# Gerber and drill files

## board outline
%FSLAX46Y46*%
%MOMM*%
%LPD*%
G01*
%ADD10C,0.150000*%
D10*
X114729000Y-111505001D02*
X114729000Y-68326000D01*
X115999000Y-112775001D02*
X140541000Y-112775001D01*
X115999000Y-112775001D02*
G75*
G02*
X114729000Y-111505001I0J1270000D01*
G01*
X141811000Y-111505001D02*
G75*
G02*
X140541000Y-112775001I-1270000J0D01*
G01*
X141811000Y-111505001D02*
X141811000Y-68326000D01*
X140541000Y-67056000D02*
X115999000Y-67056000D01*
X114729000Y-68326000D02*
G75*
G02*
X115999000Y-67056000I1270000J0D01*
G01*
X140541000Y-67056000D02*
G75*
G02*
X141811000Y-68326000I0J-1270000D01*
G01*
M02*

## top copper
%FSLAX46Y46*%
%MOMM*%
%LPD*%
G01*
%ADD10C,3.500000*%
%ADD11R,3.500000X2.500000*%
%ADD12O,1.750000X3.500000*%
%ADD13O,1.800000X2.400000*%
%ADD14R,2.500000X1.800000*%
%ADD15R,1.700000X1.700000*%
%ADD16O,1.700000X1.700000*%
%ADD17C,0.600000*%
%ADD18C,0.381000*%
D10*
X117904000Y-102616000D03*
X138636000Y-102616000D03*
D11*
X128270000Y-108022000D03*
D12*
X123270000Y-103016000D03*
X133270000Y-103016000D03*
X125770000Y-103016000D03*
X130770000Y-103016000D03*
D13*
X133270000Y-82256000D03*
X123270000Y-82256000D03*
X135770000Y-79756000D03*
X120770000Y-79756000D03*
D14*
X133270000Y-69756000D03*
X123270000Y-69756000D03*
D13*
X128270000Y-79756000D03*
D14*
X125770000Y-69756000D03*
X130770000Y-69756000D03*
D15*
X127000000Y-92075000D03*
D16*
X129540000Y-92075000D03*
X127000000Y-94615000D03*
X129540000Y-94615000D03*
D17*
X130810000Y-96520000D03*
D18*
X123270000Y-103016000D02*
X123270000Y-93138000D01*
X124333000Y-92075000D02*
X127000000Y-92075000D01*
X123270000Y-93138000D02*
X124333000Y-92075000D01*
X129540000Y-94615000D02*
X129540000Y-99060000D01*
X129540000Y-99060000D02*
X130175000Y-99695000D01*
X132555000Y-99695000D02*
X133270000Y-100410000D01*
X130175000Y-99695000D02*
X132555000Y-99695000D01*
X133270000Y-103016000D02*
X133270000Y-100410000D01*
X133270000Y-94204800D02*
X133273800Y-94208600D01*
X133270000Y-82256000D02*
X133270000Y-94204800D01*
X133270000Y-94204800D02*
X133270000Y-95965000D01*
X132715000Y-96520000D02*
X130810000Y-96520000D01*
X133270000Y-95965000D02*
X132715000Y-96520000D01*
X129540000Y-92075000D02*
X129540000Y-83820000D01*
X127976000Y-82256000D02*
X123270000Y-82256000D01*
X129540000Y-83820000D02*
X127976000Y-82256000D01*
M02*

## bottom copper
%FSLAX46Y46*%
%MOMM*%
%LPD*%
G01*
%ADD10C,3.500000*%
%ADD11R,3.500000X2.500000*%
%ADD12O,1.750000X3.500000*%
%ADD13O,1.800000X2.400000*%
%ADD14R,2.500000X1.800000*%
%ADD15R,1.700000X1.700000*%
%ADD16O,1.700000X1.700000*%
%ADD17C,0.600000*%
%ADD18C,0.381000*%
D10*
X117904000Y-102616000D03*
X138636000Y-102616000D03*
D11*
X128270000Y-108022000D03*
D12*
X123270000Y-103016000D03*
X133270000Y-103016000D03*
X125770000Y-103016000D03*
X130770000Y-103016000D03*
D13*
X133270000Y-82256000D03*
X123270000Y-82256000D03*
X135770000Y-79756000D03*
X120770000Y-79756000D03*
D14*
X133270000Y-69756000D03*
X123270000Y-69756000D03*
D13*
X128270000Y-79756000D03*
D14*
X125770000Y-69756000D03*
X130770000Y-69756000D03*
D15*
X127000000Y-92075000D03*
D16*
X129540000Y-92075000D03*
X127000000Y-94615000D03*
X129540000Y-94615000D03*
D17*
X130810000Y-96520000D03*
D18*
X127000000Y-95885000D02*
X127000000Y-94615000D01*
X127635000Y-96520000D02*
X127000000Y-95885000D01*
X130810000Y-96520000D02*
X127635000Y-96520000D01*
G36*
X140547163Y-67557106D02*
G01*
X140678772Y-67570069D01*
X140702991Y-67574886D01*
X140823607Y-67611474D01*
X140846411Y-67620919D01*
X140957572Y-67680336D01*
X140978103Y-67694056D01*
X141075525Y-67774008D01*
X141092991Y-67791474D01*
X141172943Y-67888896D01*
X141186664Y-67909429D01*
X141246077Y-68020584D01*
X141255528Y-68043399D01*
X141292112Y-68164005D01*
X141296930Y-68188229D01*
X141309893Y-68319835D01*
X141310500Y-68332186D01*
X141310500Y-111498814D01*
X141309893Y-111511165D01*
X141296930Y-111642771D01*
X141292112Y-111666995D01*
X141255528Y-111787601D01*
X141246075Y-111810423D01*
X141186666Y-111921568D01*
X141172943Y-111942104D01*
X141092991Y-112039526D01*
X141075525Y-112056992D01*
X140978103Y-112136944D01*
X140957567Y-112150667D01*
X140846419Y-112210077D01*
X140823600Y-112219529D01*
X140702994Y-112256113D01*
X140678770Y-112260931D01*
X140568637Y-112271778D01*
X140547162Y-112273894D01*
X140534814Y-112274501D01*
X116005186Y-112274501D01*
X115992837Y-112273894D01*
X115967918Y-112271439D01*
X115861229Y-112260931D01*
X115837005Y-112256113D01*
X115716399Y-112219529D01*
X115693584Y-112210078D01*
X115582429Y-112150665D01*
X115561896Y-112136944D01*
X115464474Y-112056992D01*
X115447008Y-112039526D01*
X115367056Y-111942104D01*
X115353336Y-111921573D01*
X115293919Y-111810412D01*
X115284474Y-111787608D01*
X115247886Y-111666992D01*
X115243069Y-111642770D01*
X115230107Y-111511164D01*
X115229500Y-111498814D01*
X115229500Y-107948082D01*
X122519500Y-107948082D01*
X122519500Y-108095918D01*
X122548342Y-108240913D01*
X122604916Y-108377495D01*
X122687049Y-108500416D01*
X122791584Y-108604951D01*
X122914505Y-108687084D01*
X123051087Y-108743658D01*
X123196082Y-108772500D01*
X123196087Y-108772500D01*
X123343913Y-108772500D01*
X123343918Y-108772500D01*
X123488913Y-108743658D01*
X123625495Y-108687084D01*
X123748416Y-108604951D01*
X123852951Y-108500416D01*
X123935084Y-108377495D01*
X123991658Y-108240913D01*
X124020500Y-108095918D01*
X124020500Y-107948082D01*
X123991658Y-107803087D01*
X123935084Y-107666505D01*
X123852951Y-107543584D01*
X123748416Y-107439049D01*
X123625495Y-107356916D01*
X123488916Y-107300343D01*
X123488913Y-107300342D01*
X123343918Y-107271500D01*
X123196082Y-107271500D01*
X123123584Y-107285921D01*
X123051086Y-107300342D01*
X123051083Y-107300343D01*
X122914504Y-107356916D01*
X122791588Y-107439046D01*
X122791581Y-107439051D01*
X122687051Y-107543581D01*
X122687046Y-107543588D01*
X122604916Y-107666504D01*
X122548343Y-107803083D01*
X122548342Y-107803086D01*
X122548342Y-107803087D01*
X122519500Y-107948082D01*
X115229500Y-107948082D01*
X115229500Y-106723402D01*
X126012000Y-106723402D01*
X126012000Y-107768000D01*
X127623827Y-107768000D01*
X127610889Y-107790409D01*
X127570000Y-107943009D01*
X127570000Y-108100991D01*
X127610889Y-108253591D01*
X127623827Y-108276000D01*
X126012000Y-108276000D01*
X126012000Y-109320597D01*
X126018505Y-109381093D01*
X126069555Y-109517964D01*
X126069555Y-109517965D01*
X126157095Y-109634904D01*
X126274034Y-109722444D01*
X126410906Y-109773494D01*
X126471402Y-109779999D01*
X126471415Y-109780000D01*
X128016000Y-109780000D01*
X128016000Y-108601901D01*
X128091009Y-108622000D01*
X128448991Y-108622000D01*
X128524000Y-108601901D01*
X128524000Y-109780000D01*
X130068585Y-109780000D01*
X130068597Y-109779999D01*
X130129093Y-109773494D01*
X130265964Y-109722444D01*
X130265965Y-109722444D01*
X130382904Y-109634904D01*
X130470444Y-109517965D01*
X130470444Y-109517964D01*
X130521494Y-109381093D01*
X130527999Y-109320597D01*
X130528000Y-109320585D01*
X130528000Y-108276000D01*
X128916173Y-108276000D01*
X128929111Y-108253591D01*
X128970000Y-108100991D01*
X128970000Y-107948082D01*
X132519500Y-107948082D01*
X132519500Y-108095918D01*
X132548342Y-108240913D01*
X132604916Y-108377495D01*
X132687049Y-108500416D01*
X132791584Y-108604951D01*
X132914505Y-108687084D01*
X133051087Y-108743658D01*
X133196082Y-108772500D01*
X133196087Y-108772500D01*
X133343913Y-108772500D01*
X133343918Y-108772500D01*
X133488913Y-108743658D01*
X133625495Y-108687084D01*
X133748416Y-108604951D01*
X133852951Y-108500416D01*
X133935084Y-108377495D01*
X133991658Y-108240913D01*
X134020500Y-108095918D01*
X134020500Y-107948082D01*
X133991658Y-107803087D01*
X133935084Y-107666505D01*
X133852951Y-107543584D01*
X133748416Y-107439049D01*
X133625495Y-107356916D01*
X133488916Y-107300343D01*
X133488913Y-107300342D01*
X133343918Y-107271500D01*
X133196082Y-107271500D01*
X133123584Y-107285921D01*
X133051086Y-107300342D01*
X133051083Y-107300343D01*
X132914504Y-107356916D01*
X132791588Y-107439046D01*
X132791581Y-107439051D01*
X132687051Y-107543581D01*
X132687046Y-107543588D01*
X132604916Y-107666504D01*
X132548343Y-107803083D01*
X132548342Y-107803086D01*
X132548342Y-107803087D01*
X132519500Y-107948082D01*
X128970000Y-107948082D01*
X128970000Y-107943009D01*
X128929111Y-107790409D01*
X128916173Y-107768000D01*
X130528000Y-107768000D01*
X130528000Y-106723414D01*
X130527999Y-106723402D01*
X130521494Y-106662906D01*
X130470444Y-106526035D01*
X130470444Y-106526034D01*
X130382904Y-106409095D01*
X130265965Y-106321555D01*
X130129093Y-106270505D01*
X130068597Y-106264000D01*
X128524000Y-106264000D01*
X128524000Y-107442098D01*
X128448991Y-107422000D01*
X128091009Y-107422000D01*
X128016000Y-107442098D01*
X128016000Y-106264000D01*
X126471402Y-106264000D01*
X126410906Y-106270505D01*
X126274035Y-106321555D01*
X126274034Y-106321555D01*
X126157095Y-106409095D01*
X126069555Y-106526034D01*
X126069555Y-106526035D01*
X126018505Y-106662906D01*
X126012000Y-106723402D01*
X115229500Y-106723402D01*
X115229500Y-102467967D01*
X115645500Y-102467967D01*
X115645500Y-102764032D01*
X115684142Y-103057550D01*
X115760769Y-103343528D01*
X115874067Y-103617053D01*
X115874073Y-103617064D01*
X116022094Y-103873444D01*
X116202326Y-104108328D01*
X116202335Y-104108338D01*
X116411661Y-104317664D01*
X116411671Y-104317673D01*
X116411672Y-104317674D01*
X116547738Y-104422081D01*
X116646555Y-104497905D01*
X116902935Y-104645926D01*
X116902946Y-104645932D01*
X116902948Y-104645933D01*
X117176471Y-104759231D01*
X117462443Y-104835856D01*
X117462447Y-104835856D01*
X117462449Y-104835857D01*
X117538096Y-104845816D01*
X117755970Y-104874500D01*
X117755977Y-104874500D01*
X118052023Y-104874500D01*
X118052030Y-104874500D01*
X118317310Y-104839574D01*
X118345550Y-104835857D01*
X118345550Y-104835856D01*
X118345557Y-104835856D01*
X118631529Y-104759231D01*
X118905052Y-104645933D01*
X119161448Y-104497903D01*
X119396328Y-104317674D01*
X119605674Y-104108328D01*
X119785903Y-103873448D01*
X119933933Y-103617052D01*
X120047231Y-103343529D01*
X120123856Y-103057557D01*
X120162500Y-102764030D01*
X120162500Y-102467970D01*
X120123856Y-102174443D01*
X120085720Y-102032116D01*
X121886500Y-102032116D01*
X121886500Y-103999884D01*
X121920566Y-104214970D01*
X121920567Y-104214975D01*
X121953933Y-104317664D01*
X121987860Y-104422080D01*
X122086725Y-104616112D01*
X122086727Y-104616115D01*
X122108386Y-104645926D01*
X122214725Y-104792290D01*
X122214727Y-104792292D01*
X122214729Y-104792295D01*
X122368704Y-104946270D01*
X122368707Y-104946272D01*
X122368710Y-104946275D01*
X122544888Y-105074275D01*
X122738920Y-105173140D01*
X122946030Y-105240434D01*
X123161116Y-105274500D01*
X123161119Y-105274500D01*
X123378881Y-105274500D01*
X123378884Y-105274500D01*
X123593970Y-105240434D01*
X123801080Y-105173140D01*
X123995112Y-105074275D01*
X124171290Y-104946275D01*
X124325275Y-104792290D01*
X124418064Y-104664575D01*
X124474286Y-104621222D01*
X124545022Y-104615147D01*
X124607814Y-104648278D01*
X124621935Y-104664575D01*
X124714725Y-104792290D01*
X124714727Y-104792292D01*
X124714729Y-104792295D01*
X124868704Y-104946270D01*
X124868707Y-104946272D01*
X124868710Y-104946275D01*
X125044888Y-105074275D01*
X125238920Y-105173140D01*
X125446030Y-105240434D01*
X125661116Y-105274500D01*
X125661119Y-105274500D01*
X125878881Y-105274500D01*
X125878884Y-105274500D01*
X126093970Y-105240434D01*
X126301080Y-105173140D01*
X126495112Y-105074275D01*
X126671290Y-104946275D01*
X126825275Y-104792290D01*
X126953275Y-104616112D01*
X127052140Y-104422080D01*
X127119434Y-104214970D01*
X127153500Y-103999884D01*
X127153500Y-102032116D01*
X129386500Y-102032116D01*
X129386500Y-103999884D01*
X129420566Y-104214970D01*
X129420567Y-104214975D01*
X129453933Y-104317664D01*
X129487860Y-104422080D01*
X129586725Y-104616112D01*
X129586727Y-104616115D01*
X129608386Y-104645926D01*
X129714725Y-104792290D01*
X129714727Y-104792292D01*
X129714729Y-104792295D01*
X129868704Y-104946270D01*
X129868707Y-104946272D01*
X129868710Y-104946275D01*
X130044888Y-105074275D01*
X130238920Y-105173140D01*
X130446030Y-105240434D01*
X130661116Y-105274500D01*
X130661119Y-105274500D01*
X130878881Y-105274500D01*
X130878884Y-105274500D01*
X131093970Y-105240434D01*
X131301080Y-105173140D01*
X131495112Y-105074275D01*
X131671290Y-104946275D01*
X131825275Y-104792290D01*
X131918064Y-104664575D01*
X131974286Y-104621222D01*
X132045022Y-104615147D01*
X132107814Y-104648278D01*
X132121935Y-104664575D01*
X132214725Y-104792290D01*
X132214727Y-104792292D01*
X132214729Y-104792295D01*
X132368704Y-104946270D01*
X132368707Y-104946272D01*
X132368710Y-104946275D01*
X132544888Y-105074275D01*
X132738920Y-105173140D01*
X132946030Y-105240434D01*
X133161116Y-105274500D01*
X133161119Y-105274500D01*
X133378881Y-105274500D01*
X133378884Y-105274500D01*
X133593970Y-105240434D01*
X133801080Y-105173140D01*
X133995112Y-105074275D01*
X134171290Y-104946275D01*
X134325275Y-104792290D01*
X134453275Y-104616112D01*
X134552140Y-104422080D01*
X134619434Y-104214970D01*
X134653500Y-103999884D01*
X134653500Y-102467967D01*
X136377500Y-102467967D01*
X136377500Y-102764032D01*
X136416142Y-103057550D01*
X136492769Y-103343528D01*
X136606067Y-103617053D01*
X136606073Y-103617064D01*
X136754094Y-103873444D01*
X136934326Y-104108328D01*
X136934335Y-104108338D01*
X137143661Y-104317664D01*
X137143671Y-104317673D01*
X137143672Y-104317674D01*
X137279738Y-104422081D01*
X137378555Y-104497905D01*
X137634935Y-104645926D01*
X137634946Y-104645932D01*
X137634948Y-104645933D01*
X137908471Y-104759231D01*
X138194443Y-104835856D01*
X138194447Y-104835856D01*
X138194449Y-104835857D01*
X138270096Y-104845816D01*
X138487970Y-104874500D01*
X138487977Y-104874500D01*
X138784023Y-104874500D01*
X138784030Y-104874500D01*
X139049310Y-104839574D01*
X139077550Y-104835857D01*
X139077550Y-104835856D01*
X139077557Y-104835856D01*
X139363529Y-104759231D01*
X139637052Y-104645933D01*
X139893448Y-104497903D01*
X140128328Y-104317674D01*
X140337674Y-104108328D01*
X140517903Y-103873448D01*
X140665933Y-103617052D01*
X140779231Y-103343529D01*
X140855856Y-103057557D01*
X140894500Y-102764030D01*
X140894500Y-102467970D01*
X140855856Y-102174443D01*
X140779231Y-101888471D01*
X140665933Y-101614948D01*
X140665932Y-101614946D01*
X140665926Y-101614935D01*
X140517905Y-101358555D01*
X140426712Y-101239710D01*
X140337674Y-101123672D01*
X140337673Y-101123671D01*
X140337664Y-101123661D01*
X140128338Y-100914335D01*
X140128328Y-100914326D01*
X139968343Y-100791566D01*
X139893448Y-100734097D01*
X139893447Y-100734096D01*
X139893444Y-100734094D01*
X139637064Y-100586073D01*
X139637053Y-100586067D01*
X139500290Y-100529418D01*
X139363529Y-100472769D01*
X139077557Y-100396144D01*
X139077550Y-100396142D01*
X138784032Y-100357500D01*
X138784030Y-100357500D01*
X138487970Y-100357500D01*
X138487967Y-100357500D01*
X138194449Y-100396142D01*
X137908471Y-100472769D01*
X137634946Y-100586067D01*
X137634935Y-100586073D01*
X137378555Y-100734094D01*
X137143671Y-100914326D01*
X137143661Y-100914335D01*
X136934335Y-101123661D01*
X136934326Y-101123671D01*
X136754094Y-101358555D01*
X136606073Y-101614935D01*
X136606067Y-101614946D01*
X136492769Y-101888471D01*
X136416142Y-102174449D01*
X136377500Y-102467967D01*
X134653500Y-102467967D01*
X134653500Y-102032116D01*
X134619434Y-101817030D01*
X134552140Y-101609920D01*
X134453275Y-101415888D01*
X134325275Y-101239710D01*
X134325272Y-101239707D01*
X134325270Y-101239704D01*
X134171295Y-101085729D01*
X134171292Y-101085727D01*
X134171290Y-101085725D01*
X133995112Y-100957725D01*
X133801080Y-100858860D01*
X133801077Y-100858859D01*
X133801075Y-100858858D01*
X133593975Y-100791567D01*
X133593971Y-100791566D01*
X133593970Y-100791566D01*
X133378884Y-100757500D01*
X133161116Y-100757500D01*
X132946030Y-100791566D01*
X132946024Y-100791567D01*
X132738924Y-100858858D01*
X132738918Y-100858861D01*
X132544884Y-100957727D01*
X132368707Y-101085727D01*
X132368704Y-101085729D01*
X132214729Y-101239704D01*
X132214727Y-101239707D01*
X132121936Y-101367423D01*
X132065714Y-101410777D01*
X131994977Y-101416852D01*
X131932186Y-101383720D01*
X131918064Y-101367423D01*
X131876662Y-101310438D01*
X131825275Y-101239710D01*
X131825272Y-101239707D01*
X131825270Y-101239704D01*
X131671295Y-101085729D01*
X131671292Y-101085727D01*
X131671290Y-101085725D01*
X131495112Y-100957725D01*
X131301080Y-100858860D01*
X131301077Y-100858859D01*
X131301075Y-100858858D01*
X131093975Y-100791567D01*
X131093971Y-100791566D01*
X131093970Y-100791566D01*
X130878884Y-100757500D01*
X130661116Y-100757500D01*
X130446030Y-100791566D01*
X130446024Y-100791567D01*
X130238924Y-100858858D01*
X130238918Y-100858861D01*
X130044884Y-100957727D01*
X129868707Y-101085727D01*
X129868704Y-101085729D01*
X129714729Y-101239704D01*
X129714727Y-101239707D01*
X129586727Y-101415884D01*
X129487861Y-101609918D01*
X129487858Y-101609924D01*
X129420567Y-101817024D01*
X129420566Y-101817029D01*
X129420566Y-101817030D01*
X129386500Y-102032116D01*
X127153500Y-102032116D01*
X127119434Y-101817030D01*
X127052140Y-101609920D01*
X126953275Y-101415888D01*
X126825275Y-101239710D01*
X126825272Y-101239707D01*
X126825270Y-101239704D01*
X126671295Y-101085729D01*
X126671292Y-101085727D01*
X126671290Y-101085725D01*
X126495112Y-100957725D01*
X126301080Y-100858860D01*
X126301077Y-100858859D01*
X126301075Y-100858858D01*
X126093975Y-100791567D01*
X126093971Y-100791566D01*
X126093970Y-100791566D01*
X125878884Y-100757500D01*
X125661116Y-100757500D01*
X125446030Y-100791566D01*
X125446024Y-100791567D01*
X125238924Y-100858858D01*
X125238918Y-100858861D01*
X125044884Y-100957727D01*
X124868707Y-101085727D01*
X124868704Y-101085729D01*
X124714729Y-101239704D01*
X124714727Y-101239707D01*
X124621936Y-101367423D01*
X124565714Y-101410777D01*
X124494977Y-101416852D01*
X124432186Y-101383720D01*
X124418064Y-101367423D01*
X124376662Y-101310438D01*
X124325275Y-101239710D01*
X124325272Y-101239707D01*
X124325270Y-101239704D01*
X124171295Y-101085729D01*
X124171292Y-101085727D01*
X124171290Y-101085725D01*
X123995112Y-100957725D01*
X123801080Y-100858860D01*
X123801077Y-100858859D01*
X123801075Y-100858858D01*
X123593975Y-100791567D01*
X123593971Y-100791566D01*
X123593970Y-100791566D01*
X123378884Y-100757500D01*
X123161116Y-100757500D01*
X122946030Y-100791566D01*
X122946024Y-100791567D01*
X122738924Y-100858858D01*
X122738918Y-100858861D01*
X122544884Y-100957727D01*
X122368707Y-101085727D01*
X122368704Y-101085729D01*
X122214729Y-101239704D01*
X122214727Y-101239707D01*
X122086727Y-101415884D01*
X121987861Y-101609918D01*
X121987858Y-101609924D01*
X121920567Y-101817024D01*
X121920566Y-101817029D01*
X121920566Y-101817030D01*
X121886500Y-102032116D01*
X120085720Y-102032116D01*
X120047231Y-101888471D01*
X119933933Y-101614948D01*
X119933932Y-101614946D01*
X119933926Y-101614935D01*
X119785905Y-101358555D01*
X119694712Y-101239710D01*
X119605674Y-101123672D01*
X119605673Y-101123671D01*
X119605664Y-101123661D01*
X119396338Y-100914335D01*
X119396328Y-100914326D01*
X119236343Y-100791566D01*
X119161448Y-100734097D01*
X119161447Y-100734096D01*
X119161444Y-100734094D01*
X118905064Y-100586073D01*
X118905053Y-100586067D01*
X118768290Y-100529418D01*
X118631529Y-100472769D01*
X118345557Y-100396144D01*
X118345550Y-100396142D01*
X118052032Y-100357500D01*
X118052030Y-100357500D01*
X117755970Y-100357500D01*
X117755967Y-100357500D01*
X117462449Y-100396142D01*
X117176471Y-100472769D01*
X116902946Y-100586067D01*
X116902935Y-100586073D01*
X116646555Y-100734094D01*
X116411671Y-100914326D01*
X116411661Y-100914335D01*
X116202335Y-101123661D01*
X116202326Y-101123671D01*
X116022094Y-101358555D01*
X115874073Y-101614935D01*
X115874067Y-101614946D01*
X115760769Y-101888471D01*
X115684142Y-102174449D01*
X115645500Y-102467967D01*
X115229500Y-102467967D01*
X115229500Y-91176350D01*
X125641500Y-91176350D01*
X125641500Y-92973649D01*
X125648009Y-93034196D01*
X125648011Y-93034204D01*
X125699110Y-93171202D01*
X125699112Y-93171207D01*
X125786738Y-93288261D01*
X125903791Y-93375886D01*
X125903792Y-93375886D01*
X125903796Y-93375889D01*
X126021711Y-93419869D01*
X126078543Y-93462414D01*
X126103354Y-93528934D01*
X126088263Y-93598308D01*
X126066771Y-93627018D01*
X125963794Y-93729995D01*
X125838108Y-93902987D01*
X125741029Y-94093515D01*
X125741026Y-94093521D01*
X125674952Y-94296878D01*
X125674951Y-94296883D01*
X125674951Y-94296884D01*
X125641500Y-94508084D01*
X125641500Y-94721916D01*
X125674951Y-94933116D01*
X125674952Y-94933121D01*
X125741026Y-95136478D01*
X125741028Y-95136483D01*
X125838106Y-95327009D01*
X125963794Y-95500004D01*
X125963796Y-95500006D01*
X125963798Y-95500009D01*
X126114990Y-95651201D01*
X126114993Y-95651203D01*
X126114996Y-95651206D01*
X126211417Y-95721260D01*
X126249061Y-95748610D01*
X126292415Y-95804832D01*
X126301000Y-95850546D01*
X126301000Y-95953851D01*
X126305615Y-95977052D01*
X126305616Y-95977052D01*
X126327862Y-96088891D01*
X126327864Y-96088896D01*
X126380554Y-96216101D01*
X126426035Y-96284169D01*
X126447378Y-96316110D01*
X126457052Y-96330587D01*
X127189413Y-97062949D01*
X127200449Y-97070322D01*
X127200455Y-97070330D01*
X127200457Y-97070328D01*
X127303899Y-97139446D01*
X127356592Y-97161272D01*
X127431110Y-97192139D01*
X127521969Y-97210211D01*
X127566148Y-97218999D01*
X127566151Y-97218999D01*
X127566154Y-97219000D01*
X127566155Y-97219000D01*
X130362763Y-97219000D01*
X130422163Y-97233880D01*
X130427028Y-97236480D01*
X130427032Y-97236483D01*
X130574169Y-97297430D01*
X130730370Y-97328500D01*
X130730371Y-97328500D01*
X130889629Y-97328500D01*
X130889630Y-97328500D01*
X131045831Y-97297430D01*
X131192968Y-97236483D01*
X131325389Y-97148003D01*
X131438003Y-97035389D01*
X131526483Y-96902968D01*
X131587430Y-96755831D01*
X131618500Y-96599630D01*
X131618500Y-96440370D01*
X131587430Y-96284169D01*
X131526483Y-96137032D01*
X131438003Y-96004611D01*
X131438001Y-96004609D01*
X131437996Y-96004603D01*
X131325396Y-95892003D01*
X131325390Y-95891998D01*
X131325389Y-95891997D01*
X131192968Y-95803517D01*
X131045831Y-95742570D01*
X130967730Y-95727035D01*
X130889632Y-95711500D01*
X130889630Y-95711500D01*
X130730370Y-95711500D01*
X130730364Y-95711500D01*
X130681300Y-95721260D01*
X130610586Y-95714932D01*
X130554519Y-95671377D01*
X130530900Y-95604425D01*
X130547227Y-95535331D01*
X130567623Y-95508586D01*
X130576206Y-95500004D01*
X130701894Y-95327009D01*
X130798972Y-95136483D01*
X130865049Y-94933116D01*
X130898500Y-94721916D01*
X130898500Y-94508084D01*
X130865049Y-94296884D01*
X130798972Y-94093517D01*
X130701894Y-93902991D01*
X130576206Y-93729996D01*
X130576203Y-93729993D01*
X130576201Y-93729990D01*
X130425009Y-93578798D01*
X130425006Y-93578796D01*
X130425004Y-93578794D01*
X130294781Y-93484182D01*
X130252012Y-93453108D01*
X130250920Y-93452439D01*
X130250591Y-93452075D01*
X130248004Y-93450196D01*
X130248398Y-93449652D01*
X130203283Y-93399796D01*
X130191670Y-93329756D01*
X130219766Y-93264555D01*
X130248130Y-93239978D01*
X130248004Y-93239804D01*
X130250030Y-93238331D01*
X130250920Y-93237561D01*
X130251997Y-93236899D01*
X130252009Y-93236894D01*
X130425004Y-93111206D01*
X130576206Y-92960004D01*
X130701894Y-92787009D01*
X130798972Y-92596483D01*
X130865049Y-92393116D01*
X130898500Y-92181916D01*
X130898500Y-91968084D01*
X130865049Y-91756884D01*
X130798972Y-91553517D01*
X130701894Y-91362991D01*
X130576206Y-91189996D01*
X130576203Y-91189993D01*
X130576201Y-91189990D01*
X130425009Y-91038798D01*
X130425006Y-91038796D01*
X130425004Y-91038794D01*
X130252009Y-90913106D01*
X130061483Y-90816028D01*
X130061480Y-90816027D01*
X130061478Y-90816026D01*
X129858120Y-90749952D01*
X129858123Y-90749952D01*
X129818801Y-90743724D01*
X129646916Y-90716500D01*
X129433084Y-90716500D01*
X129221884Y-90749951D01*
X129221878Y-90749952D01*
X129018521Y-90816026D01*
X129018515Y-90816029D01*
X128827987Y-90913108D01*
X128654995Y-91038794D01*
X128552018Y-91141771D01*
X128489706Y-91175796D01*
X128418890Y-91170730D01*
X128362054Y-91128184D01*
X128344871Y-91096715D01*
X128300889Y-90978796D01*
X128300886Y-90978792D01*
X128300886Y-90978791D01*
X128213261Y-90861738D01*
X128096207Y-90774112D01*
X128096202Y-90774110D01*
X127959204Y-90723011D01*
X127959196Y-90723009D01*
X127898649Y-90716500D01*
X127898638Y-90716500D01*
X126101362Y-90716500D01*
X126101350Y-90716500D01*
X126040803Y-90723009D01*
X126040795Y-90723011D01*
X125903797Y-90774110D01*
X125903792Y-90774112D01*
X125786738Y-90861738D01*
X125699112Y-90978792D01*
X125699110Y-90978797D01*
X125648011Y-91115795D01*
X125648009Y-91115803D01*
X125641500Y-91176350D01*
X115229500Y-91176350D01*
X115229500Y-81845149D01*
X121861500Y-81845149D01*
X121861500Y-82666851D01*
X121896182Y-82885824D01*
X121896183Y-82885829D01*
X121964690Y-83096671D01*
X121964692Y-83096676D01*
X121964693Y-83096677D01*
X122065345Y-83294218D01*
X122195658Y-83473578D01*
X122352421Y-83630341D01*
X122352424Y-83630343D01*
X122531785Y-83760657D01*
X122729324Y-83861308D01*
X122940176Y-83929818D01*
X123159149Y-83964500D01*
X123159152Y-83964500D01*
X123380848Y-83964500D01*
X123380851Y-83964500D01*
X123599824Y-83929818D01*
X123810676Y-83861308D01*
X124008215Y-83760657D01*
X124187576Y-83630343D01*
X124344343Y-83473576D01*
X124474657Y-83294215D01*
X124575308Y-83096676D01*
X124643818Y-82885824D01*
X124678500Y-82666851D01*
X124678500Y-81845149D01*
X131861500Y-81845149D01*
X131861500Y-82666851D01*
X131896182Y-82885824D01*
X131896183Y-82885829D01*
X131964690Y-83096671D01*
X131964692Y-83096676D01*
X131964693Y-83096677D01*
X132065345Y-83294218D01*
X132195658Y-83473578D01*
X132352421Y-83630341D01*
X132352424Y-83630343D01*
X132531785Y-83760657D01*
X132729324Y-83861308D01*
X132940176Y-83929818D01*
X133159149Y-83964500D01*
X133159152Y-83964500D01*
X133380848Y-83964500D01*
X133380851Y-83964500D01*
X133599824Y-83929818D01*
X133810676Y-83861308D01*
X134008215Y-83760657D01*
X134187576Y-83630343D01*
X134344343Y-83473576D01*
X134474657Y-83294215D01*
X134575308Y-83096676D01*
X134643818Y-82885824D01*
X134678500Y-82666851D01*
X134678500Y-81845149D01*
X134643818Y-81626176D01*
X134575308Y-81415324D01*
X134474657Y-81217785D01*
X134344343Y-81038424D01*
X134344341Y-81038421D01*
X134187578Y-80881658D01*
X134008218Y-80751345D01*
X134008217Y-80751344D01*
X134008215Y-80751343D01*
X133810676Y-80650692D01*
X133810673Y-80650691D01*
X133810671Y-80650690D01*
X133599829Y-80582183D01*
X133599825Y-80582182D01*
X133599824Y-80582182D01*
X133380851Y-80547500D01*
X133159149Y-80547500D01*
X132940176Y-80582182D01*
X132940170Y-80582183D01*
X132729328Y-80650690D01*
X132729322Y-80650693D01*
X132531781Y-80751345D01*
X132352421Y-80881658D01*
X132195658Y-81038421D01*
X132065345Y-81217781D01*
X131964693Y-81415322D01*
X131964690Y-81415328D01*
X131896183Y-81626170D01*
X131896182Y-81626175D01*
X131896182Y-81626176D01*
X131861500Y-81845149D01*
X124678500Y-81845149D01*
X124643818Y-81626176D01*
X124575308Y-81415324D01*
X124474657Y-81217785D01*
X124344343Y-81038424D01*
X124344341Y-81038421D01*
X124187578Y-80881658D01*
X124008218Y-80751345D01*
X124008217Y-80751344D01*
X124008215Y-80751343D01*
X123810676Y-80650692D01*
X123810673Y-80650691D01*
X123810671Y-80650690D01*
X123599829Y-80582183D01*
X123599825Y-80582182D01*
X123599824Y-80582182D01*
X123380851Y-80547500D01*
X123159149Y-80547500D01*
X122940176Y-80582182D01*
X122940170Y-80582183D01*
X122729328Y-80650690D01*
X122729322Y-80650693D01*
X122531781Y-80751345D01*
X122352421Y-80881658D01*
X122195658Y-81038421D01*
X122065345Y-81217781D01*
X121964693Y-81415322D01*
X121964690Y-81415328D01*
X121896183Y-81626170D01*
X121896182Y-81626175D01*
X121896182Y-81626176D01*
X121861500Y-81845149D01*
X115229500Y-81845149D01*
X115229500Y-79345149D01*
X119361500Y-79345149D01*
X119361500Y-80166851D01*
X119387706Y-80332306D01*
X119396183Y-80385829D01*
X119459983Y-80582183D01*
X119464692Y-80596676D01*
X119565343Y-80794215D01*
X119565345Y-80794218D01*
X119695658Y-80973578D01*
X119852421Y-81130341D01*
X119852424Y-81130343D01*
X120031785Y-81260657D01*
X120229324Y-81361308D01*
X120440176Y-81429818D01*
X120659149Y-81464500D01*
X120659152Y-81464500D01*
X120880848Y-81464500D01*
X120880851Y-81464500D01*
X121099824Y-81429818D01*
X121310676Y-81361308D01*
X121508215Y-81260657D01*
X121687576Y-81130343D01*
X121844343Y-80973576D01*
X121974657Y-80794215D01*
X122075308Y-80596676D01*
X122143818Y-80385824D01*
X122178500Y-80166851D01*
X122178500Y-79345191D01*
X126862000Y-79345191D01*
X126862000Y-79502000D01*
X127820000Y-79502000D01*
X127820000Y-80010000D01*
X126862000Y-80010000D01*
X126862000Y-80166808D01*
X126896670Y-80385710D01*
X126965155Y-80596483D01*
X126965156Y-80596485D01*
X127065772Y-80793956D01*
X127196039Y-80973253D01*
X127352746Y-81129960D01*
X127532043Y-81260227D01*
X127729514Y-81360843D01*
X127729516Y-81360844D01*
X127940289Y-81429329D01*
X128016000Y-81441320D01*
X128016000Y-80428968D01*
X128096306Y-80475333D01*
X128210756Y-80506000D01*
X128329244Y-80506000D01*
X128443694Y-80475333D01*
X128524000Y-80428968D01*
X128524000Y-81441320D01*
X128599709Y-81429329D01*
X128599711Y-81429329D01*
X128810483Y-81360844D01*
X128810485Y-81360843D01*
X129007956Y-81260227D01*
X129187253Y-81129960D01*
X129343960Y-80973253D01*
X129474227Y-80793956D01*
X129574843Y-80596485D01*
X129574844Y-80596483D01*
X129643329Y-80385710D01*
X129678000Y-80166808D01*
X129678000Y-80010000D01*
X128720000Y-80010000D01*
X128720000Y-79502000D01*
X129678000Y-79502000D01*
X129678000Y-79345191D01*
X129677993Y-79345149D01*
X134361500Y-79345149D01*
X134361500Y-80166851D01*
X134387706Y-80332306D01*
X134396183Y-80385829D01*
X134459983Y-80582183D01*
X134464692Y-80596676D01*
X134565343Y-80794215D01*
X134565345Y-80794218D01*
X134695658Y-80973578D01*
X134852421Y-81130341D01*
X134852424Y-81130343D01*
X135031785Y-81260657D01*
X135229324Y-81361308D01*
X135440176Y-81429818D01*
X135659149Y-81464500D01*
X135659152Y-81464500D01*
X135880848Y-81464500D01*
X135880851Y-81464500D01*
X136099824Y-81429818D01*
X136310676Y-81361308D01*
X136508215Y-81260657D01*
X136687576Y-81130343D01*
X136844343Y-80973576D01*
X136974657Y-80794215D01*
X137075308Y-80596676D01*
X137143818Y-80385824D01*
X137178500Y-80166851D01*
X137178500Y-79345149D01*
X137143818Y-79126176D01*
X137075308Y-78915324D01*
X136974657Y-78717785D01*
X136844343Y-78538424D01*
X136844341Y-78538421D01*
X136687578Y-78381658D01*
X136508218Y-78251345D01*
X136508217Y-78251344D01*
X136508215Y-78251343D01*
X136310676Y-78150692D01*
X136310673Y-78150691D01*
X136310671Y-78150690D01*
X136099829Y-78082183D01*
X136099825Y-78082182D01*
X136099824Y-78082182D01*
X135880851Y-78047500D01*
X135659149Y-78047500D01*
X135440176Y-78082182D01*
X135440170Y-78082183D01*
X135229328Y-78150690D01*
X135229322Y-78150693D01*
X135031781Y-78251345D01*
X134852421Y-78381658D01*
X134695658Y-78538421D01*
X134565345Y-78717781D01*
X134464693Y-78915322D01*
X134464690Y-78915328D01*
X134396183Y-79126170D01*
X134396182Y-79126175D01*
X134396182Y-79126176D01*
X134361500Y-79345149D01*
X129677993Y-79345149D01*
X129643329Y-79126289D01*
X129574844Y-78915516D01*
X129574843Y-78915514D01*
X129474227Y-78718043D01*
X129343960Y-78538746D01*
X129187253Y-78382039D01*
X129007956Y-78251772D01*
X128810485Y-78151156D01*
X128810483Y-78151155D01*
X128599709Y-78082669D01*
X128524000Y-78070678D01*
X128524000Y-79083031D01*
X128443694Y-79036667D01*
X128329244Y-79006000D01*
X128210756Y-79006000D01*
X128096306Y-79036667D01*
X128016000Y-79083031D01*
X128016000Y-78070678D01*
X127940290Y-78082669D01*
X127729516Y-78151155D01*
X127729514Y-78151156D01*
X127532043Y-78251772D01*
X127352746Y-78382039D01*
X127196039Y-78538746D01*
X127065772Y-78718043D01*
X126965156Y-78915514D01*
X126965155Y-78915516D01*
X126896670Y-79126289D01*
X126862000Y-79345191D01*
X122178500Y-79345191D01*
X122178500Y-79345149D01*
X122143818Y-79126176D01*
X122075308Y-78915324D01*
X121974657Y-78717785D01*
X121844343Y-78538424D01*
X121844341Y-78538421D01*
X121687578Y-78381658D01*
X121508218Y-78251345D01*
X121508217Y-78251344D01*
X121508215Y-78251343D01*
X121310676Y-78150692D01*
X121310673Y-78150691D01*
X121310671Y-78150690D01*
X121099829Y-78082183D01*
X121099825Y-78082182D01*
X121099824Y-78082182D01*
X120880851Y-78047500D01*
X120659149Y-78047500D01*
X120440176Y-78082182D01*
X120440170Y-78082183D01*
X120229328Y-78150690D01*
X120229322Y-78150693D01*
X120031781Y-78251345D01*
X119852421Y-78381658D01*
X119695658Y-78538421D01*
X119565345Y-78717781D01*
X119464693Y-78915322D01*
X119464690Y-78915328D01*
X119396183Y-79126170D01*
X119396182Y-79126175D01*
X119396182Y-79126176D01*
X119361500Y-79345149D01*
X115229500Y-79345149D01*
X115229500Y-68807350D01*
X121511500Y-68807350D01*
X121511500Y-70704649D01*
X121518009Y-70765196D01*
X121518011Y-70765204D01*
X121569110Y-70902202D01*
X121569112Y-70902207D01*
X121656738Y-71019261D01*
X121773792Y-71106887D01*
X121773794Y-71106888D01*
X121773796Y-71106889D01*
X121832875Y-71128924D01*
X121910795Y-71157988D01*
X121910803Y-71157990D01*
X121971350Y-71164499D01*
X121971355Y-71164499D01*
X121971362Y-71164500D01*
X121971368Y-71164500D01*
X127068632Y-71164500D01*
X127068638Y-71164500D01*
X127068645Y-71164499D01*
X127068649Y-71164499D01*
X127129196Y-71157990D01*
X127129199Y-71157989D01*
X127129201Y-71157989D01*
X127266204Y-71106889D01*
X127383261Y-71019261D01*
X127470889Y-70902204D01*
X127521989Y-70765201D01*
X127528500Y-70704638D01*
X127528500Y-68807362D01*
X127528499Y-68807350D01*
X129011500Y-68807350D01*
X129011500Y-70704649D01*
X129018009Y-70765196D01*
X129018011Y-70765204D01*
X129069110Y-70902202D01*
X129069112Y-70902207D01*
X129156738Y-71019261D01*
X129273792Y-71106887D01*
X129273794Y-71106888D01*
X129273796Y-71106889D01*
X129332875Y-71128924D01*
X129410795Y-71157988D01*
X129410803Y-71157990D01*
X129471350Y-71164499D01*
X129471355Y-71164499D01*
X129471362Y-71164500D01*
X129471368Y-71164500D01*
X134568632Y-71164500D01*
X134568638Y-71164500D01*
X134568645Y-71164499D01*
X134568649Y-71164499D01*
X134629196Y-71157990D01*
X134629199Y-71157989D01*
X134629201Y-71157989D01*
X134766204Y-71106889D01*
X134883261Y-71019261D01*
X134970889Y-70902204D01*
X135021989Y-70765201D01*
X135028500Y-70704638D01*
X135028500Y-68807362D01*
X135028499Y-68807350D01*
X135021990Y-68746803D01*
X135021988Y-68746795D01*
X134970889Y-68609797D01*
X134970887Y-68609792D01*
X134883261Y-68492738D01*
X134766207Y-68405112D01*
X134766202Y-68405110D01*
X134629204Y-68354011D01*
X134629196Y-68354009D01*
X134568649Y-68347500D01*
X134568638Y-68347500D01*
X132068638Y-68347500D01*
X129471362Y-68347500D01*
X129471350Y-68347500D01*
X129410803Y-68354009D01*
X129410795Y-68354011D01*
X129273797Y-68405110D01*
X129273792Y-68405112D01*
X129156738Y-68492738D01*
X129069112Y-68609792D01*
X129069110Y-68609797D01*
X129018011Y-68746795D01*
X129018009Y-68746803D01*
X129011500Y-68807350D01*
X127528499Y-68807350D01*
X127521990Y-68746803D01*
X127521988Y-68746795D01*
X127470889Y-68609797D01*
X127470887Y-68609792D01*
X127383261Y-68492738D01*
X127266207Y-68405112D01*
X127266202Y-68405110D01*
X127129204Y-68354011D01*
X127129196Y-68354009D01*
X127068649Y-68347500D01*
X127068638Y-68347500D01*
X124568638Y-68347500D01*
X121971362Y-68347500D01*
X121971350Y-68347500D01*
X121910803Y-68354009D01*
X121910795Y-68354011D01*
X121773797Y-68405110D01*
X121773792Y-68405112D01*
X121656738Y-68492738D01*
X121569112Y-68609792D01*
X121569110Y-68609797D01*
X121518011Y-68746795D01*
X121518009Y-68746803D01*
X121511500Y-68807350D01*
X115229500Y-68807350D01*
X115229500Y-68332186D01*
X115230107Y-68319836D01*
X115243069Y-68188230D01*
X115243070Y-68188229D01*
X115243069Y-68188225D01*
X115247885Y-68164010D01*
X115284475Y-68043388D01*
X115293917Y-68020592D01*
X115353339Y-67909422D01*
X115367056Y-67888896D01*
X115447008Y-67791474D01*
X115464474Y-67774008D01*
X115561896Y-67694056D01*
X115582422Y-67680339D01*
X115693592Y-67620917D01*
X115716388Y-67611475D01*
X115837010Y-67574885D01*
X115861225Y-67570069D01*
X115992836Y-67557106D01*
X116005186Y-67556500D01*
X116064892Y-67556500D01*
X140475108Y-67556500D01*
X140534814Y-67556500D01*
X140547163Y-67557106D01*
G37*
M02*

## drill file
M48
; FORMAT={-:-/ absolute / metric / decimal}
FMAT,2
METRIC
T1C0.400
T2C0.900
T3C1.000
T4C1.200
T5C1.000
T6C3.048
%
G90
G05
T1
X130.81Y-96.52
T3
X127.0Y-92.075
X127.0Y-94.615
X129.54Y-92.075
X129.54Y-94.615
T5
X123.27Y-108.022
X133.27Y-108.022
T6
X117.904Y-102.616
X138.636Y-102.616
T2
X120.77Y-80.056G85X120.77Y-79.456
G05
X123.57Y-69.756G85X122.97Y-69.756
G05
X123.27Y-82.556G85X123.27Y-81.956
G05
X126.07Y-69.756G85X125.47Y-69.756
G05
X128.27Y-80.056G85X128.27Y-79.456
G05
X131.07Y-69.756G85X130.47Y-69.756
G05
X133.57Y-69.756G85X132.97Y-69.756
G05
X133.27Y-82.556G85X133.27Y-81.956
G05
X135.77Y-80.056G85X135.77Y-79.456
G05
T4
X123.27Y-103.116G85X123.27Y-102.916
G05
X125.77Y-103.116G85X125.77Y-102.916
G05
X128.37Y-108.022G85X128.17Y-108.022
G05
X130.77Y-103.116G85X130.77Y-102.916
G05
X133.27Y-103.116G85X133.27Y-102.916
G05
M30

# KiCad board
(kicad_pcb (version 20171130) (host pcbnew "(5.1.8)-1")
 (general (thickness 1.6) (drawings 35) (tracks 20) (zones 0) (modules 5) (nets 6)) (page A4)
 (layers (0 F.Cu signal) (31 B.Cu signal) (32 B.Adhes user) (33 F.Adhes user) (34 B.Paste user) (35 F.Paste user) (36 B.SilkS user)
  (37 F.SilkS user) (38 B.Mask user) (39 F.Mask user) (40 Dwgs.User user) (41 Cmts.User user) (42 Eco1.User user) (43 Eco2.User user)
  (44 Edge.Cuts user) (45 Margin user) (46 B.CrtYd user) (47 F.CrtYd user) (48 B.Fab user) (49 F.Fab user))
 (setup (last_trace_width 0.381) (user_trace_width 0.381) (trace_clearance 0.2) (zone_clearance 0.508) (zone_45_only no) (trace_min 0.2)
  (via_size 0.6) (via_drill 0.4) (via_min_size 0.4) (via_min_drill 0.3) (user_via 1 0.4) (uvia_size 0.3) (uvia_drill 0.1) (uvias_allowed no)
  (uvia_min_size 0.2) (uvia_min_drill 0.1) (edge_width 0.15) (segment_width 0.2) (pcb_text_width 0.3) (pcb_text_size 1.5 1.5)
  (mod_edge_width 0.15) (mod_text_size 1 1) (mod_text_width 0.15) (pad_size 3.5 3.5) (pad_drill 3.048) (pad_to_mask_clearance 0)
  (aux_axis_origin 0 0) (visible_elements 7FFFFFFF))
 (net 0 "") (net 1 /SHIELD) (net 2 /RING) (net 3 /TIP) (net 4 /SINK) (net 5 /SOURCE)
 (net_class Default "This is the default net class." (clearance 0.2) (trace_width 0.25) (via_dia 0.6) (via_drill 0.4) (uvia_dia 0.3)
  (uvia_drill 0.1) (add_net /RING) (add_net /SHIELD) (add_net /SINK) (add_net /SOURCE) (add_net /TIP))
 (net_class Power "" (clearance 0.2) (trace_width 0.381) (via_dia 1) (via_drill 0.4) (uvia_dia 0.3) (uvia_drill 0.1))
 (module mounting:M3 (layer F.Cu) (at 117.904 102.616)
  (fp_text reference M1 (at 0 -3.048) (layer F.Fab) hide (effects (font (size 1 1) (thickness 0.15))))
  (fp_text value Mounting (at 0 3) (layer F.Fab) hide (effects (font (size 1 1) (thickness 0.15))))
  (pad "" np_thru_hole circle (at 0 0) (size 3.5 3.5) (drill 3.048) (layers *.Cu *.Mask) (solder_mask_margin 0.8)))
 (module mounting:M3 (layer F.Cu) (at 138.636 102.616)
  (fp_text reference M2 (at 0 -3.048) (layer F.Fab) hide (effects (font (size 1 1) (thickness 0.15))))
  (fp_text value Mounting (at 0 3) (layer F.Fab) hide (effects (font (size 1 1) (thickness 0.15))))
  (pad "" np_thru_hole circle (at 0 0) (size 3.5 3.5) (drill 3.048) (layers *.Cu *.Mask) (solder_mask_margin 0.8)))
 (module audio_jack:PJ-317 (layer F.Cu) (at 128.27 106.426 180)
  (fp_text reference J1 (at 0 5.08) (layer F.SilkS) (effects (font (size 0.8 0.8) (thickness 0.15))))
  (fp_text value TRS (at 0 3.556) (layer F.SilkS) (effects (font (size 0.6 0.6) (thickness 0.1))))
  (pad 1 thru_hole rect (at 0 -1.596 180) (size 3.5 2.5) (drill oval 1.4 1.2) (layers *.Cu *.Mask) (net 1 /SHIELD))
  (pad 2 thru_hole oval (at 5 3.41 180) (size 1.75 3.5) (drill oval 1.2 1.4) (layers *.Cu *.Mask) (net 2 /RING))
  (pad 5 thru_hole oval (at -5 3.41 180) (size 1.75 3.5) (drill oval 1.2 1.4) (layers *.Cu *.Mask) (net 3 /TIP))
  (pad 3 thru_hole oval (at 2.5 3.41 180) (size 1.75 3.5) (drill oval 1.2 1.4) (layers *.Cu *.Mask))
  (pad 4 thru_hole oval (at -2.5 3.41 180) (size 1.75 3.5) (drill oval 1.2 1.4) (layers *.Cu *.Mask))
  (pad "" np_thru_hole circle (at -5 -1.596 180) (size 1 1) (drill 1) (layers *.Cu *.Mask))
  (pad "" np_thru_hole circle (at 5 -1.596) (size 1 1) (drill 1) (layers *.Cu *.Mask)))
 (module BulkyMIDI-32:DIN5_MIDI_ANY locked (layer F.Cu) (at 128.27 79.756 180)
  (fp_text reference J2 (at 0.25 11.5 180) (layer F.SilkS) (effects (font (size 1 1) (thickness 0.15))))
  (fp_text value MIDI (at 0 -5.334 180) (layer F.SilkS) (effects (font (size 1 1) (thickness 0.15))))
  (pad 5 thru_hole oval (at -5 -2.5 180) (size 1.8 2.4) (drill oval 0.9 1.5) (layers *.Cu *.Mask) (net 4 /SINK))
  (pad 4 thru_hole oval (at 5 -2.5 180) (size 1.8 2.4) (drill oval 0.9 1.5) (layers *.Cu *.Mask) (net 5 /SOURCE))
  (pad 3 thru_hole oval (at -7.5 0 180) (size 1.8 2.4) (drill oval 0.9 1.5) (layers *.Cu *.Mask))
  (pad 1 thru_hole oval (at 7.5 0 180) (size 1.8 2.4) (drill oval 0.9 1.5) (layers *.Cu *.Mask))
  (pad 6 thru_hole rect (at -5 10 180) (size 2.5 1.8) (drill oval 1.5 0.9) (layers *.Cu *.Mask))
  (pad 6 thru_hole rect (at 5 10 180) (size 2.5 1.8) (drill oval 1.5 0.9) (layers *.Cu *.Mask))
  (pad 2 thru_hole oval (at 0 0 180) (size 1.8 2.4) (drill oval 0.9 1.5) (layers *.Cu *.Mask) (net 1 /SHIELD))
  (pad 6 thru_hole rect (at 2.5 10 180) (size 2.5 1.8) (drill oval 1.5 0.9) (layers *.Cu *.Mask))
  (pad 6 thru_hole rect (at -2.5 10 180) (size 2.5 1.8) (drill oval 1.5 0.9) (layers *.Cu *.Mask)))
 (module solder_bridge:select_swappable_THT (layer F.Cu) (at 127 92.075)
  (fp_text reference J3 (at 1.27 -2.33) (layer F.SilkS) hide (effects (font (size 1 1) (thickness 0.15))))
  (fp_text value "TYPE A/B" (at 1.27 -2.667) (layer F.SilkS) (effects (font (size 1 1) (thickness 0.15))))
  (pad 1a thru_hole rect (at 0 0) (size 1.7 1.7) (drill 1) (layers *.Cu *.Mask) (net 2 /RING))
  (pad 1b thru_hole oval (at 2.54 0) (size 1.7 1.7) (drill 1) (layers *.Cu *.Mask) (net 5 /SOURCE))
  (pad 2b thru_hole oval (at 0 2.54) (size 1.7 1.7) (drill 1) (layers *.Cu *.Mask) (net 4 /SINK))
  (pad 2a thru_hole oval (at 2.54 2.54) (size 1.7 1.7) (drill 1) (layers *.Cu *.Mask) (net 3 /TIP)))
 (gr_line (start 114.729 111.505001) (end 114.729 68.326) (layer Edge.Cuts) (width 0.15))
 (gr_line (start 115.999 112.775001) (end 140.541 112.775001) (angle 90) (layer Edge.Cuts) (width 0.15))
 (gr_arc (start 115.999 111.505001) (end 115.999 112.775001) (angle 90) (layer Edge.Cuts) (width 0.15))
 (gr_arc (start 140.541 111.505001) (end 141.811 111.505001) (angle 90) (layer Edge.Cuts) (width 0.15))
 (gr_line (start 141.811 111.505001) (end 141.811 68.326) (layer Edge.Cuts) (width 0.15))
 (gr_line (start 140.541 67.056) (end 115.999 67.056) (angle 90) (layer Edge.Cuts) (width 0.15))
 (gr_arc (start 115.999 68.326) (end 114.729 68.326) (angle 90) (layer Edge.Cuts) (width 0.15))
 (gr_arc (start 140.541 68.326) (end 140.541 67.056) (angle 90) (layer Edge.Cuts) (width 0.15))
 (segment (start 123.27 103.016) (end 123.27 93.138) (width 0.381) (layer F.Cu) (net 2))
 (segment (start 124.333 92.075) (end 127 92.075) (width 0.381) (layer F.Cu) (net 2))
 (segment (start 123.27 93.138) (end 124.333 92.075) (width 0.381) (layer F.Cu) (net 2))
 (segment (start 129.54 94.615) (end 129.54 99.06) (width 0.381) (layer F.Cu) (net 3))
 (segment (start 129.54 99.06) (end 130.175 99.695) (width 0.381) (layer F.Cu) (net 3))
 (segment (start 132.555 99.695) (end 133.27 100.41) (width 0.381) (layer F.Cu) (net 3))
 (segment (start 130.175 99.695) (end 132.555 99.695) (width 0.381) (layer F.Cu) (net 3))
 (segment (start 133.27 103.016) (end 133.27 100.41) (width 0.381) (layer F.Cu) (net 3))
 (segment (start 133.27 94.2048) (end 133.2738 94.2086) (width 0.381) (layer F.Cu) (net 4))
 (segment (start 133.27 82.256) (end 133.27 94.2048) (width 0.381) (layer F.Cu) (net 4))
 (segment (start 127 95.885) (end 127 94.615) (width 0.381) (layer B.Cu) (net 4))
 (segment (start 127.635 96.52) (end 127 95.885) (width 0.381) (layer B.Cu) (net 4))
 (via (at 130.81 96.52) (size 0.6) (drill 0.4) (layers F.Cu B.Cu) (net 4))
 (segment (start 130.81 96.52) (end 127.635 96.52) (width 0.381) (layer B.Cu) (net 4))
 (segment (start 133.27 94.2048) (end 133.27 95.965) (width 0.381) (layer F.Cu) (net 4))
 (segment (start 132.715 96.52) (end 130.81 96.52) (width 0.381) (layer F.Cu) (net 4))
 (segment (start 133.27 95.965) (end 132.715 96.52) (width 0.381) (layer F.Cu) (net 4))
 (segment (start 129.54 92.075) (end 129.54 83.82) (width 0.381) (layer F.Cu) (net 5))
 (segment (start 127.976 82.256) (end 123.27 82.256) (width 0.381) (layer F.Cu) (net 5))
 (segment (start 129.54 83.82) (end 127.976 82.256) (width 0.381) (layer F.Cu) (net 5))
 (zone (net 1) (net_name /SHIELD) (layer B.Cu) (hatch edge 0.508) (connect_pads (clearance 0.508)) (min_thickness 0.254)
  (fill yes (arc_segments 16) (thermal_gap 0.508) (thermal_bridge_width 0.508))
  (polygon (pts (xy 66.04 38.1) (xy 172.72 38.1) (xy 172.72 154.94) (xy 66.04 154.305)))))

